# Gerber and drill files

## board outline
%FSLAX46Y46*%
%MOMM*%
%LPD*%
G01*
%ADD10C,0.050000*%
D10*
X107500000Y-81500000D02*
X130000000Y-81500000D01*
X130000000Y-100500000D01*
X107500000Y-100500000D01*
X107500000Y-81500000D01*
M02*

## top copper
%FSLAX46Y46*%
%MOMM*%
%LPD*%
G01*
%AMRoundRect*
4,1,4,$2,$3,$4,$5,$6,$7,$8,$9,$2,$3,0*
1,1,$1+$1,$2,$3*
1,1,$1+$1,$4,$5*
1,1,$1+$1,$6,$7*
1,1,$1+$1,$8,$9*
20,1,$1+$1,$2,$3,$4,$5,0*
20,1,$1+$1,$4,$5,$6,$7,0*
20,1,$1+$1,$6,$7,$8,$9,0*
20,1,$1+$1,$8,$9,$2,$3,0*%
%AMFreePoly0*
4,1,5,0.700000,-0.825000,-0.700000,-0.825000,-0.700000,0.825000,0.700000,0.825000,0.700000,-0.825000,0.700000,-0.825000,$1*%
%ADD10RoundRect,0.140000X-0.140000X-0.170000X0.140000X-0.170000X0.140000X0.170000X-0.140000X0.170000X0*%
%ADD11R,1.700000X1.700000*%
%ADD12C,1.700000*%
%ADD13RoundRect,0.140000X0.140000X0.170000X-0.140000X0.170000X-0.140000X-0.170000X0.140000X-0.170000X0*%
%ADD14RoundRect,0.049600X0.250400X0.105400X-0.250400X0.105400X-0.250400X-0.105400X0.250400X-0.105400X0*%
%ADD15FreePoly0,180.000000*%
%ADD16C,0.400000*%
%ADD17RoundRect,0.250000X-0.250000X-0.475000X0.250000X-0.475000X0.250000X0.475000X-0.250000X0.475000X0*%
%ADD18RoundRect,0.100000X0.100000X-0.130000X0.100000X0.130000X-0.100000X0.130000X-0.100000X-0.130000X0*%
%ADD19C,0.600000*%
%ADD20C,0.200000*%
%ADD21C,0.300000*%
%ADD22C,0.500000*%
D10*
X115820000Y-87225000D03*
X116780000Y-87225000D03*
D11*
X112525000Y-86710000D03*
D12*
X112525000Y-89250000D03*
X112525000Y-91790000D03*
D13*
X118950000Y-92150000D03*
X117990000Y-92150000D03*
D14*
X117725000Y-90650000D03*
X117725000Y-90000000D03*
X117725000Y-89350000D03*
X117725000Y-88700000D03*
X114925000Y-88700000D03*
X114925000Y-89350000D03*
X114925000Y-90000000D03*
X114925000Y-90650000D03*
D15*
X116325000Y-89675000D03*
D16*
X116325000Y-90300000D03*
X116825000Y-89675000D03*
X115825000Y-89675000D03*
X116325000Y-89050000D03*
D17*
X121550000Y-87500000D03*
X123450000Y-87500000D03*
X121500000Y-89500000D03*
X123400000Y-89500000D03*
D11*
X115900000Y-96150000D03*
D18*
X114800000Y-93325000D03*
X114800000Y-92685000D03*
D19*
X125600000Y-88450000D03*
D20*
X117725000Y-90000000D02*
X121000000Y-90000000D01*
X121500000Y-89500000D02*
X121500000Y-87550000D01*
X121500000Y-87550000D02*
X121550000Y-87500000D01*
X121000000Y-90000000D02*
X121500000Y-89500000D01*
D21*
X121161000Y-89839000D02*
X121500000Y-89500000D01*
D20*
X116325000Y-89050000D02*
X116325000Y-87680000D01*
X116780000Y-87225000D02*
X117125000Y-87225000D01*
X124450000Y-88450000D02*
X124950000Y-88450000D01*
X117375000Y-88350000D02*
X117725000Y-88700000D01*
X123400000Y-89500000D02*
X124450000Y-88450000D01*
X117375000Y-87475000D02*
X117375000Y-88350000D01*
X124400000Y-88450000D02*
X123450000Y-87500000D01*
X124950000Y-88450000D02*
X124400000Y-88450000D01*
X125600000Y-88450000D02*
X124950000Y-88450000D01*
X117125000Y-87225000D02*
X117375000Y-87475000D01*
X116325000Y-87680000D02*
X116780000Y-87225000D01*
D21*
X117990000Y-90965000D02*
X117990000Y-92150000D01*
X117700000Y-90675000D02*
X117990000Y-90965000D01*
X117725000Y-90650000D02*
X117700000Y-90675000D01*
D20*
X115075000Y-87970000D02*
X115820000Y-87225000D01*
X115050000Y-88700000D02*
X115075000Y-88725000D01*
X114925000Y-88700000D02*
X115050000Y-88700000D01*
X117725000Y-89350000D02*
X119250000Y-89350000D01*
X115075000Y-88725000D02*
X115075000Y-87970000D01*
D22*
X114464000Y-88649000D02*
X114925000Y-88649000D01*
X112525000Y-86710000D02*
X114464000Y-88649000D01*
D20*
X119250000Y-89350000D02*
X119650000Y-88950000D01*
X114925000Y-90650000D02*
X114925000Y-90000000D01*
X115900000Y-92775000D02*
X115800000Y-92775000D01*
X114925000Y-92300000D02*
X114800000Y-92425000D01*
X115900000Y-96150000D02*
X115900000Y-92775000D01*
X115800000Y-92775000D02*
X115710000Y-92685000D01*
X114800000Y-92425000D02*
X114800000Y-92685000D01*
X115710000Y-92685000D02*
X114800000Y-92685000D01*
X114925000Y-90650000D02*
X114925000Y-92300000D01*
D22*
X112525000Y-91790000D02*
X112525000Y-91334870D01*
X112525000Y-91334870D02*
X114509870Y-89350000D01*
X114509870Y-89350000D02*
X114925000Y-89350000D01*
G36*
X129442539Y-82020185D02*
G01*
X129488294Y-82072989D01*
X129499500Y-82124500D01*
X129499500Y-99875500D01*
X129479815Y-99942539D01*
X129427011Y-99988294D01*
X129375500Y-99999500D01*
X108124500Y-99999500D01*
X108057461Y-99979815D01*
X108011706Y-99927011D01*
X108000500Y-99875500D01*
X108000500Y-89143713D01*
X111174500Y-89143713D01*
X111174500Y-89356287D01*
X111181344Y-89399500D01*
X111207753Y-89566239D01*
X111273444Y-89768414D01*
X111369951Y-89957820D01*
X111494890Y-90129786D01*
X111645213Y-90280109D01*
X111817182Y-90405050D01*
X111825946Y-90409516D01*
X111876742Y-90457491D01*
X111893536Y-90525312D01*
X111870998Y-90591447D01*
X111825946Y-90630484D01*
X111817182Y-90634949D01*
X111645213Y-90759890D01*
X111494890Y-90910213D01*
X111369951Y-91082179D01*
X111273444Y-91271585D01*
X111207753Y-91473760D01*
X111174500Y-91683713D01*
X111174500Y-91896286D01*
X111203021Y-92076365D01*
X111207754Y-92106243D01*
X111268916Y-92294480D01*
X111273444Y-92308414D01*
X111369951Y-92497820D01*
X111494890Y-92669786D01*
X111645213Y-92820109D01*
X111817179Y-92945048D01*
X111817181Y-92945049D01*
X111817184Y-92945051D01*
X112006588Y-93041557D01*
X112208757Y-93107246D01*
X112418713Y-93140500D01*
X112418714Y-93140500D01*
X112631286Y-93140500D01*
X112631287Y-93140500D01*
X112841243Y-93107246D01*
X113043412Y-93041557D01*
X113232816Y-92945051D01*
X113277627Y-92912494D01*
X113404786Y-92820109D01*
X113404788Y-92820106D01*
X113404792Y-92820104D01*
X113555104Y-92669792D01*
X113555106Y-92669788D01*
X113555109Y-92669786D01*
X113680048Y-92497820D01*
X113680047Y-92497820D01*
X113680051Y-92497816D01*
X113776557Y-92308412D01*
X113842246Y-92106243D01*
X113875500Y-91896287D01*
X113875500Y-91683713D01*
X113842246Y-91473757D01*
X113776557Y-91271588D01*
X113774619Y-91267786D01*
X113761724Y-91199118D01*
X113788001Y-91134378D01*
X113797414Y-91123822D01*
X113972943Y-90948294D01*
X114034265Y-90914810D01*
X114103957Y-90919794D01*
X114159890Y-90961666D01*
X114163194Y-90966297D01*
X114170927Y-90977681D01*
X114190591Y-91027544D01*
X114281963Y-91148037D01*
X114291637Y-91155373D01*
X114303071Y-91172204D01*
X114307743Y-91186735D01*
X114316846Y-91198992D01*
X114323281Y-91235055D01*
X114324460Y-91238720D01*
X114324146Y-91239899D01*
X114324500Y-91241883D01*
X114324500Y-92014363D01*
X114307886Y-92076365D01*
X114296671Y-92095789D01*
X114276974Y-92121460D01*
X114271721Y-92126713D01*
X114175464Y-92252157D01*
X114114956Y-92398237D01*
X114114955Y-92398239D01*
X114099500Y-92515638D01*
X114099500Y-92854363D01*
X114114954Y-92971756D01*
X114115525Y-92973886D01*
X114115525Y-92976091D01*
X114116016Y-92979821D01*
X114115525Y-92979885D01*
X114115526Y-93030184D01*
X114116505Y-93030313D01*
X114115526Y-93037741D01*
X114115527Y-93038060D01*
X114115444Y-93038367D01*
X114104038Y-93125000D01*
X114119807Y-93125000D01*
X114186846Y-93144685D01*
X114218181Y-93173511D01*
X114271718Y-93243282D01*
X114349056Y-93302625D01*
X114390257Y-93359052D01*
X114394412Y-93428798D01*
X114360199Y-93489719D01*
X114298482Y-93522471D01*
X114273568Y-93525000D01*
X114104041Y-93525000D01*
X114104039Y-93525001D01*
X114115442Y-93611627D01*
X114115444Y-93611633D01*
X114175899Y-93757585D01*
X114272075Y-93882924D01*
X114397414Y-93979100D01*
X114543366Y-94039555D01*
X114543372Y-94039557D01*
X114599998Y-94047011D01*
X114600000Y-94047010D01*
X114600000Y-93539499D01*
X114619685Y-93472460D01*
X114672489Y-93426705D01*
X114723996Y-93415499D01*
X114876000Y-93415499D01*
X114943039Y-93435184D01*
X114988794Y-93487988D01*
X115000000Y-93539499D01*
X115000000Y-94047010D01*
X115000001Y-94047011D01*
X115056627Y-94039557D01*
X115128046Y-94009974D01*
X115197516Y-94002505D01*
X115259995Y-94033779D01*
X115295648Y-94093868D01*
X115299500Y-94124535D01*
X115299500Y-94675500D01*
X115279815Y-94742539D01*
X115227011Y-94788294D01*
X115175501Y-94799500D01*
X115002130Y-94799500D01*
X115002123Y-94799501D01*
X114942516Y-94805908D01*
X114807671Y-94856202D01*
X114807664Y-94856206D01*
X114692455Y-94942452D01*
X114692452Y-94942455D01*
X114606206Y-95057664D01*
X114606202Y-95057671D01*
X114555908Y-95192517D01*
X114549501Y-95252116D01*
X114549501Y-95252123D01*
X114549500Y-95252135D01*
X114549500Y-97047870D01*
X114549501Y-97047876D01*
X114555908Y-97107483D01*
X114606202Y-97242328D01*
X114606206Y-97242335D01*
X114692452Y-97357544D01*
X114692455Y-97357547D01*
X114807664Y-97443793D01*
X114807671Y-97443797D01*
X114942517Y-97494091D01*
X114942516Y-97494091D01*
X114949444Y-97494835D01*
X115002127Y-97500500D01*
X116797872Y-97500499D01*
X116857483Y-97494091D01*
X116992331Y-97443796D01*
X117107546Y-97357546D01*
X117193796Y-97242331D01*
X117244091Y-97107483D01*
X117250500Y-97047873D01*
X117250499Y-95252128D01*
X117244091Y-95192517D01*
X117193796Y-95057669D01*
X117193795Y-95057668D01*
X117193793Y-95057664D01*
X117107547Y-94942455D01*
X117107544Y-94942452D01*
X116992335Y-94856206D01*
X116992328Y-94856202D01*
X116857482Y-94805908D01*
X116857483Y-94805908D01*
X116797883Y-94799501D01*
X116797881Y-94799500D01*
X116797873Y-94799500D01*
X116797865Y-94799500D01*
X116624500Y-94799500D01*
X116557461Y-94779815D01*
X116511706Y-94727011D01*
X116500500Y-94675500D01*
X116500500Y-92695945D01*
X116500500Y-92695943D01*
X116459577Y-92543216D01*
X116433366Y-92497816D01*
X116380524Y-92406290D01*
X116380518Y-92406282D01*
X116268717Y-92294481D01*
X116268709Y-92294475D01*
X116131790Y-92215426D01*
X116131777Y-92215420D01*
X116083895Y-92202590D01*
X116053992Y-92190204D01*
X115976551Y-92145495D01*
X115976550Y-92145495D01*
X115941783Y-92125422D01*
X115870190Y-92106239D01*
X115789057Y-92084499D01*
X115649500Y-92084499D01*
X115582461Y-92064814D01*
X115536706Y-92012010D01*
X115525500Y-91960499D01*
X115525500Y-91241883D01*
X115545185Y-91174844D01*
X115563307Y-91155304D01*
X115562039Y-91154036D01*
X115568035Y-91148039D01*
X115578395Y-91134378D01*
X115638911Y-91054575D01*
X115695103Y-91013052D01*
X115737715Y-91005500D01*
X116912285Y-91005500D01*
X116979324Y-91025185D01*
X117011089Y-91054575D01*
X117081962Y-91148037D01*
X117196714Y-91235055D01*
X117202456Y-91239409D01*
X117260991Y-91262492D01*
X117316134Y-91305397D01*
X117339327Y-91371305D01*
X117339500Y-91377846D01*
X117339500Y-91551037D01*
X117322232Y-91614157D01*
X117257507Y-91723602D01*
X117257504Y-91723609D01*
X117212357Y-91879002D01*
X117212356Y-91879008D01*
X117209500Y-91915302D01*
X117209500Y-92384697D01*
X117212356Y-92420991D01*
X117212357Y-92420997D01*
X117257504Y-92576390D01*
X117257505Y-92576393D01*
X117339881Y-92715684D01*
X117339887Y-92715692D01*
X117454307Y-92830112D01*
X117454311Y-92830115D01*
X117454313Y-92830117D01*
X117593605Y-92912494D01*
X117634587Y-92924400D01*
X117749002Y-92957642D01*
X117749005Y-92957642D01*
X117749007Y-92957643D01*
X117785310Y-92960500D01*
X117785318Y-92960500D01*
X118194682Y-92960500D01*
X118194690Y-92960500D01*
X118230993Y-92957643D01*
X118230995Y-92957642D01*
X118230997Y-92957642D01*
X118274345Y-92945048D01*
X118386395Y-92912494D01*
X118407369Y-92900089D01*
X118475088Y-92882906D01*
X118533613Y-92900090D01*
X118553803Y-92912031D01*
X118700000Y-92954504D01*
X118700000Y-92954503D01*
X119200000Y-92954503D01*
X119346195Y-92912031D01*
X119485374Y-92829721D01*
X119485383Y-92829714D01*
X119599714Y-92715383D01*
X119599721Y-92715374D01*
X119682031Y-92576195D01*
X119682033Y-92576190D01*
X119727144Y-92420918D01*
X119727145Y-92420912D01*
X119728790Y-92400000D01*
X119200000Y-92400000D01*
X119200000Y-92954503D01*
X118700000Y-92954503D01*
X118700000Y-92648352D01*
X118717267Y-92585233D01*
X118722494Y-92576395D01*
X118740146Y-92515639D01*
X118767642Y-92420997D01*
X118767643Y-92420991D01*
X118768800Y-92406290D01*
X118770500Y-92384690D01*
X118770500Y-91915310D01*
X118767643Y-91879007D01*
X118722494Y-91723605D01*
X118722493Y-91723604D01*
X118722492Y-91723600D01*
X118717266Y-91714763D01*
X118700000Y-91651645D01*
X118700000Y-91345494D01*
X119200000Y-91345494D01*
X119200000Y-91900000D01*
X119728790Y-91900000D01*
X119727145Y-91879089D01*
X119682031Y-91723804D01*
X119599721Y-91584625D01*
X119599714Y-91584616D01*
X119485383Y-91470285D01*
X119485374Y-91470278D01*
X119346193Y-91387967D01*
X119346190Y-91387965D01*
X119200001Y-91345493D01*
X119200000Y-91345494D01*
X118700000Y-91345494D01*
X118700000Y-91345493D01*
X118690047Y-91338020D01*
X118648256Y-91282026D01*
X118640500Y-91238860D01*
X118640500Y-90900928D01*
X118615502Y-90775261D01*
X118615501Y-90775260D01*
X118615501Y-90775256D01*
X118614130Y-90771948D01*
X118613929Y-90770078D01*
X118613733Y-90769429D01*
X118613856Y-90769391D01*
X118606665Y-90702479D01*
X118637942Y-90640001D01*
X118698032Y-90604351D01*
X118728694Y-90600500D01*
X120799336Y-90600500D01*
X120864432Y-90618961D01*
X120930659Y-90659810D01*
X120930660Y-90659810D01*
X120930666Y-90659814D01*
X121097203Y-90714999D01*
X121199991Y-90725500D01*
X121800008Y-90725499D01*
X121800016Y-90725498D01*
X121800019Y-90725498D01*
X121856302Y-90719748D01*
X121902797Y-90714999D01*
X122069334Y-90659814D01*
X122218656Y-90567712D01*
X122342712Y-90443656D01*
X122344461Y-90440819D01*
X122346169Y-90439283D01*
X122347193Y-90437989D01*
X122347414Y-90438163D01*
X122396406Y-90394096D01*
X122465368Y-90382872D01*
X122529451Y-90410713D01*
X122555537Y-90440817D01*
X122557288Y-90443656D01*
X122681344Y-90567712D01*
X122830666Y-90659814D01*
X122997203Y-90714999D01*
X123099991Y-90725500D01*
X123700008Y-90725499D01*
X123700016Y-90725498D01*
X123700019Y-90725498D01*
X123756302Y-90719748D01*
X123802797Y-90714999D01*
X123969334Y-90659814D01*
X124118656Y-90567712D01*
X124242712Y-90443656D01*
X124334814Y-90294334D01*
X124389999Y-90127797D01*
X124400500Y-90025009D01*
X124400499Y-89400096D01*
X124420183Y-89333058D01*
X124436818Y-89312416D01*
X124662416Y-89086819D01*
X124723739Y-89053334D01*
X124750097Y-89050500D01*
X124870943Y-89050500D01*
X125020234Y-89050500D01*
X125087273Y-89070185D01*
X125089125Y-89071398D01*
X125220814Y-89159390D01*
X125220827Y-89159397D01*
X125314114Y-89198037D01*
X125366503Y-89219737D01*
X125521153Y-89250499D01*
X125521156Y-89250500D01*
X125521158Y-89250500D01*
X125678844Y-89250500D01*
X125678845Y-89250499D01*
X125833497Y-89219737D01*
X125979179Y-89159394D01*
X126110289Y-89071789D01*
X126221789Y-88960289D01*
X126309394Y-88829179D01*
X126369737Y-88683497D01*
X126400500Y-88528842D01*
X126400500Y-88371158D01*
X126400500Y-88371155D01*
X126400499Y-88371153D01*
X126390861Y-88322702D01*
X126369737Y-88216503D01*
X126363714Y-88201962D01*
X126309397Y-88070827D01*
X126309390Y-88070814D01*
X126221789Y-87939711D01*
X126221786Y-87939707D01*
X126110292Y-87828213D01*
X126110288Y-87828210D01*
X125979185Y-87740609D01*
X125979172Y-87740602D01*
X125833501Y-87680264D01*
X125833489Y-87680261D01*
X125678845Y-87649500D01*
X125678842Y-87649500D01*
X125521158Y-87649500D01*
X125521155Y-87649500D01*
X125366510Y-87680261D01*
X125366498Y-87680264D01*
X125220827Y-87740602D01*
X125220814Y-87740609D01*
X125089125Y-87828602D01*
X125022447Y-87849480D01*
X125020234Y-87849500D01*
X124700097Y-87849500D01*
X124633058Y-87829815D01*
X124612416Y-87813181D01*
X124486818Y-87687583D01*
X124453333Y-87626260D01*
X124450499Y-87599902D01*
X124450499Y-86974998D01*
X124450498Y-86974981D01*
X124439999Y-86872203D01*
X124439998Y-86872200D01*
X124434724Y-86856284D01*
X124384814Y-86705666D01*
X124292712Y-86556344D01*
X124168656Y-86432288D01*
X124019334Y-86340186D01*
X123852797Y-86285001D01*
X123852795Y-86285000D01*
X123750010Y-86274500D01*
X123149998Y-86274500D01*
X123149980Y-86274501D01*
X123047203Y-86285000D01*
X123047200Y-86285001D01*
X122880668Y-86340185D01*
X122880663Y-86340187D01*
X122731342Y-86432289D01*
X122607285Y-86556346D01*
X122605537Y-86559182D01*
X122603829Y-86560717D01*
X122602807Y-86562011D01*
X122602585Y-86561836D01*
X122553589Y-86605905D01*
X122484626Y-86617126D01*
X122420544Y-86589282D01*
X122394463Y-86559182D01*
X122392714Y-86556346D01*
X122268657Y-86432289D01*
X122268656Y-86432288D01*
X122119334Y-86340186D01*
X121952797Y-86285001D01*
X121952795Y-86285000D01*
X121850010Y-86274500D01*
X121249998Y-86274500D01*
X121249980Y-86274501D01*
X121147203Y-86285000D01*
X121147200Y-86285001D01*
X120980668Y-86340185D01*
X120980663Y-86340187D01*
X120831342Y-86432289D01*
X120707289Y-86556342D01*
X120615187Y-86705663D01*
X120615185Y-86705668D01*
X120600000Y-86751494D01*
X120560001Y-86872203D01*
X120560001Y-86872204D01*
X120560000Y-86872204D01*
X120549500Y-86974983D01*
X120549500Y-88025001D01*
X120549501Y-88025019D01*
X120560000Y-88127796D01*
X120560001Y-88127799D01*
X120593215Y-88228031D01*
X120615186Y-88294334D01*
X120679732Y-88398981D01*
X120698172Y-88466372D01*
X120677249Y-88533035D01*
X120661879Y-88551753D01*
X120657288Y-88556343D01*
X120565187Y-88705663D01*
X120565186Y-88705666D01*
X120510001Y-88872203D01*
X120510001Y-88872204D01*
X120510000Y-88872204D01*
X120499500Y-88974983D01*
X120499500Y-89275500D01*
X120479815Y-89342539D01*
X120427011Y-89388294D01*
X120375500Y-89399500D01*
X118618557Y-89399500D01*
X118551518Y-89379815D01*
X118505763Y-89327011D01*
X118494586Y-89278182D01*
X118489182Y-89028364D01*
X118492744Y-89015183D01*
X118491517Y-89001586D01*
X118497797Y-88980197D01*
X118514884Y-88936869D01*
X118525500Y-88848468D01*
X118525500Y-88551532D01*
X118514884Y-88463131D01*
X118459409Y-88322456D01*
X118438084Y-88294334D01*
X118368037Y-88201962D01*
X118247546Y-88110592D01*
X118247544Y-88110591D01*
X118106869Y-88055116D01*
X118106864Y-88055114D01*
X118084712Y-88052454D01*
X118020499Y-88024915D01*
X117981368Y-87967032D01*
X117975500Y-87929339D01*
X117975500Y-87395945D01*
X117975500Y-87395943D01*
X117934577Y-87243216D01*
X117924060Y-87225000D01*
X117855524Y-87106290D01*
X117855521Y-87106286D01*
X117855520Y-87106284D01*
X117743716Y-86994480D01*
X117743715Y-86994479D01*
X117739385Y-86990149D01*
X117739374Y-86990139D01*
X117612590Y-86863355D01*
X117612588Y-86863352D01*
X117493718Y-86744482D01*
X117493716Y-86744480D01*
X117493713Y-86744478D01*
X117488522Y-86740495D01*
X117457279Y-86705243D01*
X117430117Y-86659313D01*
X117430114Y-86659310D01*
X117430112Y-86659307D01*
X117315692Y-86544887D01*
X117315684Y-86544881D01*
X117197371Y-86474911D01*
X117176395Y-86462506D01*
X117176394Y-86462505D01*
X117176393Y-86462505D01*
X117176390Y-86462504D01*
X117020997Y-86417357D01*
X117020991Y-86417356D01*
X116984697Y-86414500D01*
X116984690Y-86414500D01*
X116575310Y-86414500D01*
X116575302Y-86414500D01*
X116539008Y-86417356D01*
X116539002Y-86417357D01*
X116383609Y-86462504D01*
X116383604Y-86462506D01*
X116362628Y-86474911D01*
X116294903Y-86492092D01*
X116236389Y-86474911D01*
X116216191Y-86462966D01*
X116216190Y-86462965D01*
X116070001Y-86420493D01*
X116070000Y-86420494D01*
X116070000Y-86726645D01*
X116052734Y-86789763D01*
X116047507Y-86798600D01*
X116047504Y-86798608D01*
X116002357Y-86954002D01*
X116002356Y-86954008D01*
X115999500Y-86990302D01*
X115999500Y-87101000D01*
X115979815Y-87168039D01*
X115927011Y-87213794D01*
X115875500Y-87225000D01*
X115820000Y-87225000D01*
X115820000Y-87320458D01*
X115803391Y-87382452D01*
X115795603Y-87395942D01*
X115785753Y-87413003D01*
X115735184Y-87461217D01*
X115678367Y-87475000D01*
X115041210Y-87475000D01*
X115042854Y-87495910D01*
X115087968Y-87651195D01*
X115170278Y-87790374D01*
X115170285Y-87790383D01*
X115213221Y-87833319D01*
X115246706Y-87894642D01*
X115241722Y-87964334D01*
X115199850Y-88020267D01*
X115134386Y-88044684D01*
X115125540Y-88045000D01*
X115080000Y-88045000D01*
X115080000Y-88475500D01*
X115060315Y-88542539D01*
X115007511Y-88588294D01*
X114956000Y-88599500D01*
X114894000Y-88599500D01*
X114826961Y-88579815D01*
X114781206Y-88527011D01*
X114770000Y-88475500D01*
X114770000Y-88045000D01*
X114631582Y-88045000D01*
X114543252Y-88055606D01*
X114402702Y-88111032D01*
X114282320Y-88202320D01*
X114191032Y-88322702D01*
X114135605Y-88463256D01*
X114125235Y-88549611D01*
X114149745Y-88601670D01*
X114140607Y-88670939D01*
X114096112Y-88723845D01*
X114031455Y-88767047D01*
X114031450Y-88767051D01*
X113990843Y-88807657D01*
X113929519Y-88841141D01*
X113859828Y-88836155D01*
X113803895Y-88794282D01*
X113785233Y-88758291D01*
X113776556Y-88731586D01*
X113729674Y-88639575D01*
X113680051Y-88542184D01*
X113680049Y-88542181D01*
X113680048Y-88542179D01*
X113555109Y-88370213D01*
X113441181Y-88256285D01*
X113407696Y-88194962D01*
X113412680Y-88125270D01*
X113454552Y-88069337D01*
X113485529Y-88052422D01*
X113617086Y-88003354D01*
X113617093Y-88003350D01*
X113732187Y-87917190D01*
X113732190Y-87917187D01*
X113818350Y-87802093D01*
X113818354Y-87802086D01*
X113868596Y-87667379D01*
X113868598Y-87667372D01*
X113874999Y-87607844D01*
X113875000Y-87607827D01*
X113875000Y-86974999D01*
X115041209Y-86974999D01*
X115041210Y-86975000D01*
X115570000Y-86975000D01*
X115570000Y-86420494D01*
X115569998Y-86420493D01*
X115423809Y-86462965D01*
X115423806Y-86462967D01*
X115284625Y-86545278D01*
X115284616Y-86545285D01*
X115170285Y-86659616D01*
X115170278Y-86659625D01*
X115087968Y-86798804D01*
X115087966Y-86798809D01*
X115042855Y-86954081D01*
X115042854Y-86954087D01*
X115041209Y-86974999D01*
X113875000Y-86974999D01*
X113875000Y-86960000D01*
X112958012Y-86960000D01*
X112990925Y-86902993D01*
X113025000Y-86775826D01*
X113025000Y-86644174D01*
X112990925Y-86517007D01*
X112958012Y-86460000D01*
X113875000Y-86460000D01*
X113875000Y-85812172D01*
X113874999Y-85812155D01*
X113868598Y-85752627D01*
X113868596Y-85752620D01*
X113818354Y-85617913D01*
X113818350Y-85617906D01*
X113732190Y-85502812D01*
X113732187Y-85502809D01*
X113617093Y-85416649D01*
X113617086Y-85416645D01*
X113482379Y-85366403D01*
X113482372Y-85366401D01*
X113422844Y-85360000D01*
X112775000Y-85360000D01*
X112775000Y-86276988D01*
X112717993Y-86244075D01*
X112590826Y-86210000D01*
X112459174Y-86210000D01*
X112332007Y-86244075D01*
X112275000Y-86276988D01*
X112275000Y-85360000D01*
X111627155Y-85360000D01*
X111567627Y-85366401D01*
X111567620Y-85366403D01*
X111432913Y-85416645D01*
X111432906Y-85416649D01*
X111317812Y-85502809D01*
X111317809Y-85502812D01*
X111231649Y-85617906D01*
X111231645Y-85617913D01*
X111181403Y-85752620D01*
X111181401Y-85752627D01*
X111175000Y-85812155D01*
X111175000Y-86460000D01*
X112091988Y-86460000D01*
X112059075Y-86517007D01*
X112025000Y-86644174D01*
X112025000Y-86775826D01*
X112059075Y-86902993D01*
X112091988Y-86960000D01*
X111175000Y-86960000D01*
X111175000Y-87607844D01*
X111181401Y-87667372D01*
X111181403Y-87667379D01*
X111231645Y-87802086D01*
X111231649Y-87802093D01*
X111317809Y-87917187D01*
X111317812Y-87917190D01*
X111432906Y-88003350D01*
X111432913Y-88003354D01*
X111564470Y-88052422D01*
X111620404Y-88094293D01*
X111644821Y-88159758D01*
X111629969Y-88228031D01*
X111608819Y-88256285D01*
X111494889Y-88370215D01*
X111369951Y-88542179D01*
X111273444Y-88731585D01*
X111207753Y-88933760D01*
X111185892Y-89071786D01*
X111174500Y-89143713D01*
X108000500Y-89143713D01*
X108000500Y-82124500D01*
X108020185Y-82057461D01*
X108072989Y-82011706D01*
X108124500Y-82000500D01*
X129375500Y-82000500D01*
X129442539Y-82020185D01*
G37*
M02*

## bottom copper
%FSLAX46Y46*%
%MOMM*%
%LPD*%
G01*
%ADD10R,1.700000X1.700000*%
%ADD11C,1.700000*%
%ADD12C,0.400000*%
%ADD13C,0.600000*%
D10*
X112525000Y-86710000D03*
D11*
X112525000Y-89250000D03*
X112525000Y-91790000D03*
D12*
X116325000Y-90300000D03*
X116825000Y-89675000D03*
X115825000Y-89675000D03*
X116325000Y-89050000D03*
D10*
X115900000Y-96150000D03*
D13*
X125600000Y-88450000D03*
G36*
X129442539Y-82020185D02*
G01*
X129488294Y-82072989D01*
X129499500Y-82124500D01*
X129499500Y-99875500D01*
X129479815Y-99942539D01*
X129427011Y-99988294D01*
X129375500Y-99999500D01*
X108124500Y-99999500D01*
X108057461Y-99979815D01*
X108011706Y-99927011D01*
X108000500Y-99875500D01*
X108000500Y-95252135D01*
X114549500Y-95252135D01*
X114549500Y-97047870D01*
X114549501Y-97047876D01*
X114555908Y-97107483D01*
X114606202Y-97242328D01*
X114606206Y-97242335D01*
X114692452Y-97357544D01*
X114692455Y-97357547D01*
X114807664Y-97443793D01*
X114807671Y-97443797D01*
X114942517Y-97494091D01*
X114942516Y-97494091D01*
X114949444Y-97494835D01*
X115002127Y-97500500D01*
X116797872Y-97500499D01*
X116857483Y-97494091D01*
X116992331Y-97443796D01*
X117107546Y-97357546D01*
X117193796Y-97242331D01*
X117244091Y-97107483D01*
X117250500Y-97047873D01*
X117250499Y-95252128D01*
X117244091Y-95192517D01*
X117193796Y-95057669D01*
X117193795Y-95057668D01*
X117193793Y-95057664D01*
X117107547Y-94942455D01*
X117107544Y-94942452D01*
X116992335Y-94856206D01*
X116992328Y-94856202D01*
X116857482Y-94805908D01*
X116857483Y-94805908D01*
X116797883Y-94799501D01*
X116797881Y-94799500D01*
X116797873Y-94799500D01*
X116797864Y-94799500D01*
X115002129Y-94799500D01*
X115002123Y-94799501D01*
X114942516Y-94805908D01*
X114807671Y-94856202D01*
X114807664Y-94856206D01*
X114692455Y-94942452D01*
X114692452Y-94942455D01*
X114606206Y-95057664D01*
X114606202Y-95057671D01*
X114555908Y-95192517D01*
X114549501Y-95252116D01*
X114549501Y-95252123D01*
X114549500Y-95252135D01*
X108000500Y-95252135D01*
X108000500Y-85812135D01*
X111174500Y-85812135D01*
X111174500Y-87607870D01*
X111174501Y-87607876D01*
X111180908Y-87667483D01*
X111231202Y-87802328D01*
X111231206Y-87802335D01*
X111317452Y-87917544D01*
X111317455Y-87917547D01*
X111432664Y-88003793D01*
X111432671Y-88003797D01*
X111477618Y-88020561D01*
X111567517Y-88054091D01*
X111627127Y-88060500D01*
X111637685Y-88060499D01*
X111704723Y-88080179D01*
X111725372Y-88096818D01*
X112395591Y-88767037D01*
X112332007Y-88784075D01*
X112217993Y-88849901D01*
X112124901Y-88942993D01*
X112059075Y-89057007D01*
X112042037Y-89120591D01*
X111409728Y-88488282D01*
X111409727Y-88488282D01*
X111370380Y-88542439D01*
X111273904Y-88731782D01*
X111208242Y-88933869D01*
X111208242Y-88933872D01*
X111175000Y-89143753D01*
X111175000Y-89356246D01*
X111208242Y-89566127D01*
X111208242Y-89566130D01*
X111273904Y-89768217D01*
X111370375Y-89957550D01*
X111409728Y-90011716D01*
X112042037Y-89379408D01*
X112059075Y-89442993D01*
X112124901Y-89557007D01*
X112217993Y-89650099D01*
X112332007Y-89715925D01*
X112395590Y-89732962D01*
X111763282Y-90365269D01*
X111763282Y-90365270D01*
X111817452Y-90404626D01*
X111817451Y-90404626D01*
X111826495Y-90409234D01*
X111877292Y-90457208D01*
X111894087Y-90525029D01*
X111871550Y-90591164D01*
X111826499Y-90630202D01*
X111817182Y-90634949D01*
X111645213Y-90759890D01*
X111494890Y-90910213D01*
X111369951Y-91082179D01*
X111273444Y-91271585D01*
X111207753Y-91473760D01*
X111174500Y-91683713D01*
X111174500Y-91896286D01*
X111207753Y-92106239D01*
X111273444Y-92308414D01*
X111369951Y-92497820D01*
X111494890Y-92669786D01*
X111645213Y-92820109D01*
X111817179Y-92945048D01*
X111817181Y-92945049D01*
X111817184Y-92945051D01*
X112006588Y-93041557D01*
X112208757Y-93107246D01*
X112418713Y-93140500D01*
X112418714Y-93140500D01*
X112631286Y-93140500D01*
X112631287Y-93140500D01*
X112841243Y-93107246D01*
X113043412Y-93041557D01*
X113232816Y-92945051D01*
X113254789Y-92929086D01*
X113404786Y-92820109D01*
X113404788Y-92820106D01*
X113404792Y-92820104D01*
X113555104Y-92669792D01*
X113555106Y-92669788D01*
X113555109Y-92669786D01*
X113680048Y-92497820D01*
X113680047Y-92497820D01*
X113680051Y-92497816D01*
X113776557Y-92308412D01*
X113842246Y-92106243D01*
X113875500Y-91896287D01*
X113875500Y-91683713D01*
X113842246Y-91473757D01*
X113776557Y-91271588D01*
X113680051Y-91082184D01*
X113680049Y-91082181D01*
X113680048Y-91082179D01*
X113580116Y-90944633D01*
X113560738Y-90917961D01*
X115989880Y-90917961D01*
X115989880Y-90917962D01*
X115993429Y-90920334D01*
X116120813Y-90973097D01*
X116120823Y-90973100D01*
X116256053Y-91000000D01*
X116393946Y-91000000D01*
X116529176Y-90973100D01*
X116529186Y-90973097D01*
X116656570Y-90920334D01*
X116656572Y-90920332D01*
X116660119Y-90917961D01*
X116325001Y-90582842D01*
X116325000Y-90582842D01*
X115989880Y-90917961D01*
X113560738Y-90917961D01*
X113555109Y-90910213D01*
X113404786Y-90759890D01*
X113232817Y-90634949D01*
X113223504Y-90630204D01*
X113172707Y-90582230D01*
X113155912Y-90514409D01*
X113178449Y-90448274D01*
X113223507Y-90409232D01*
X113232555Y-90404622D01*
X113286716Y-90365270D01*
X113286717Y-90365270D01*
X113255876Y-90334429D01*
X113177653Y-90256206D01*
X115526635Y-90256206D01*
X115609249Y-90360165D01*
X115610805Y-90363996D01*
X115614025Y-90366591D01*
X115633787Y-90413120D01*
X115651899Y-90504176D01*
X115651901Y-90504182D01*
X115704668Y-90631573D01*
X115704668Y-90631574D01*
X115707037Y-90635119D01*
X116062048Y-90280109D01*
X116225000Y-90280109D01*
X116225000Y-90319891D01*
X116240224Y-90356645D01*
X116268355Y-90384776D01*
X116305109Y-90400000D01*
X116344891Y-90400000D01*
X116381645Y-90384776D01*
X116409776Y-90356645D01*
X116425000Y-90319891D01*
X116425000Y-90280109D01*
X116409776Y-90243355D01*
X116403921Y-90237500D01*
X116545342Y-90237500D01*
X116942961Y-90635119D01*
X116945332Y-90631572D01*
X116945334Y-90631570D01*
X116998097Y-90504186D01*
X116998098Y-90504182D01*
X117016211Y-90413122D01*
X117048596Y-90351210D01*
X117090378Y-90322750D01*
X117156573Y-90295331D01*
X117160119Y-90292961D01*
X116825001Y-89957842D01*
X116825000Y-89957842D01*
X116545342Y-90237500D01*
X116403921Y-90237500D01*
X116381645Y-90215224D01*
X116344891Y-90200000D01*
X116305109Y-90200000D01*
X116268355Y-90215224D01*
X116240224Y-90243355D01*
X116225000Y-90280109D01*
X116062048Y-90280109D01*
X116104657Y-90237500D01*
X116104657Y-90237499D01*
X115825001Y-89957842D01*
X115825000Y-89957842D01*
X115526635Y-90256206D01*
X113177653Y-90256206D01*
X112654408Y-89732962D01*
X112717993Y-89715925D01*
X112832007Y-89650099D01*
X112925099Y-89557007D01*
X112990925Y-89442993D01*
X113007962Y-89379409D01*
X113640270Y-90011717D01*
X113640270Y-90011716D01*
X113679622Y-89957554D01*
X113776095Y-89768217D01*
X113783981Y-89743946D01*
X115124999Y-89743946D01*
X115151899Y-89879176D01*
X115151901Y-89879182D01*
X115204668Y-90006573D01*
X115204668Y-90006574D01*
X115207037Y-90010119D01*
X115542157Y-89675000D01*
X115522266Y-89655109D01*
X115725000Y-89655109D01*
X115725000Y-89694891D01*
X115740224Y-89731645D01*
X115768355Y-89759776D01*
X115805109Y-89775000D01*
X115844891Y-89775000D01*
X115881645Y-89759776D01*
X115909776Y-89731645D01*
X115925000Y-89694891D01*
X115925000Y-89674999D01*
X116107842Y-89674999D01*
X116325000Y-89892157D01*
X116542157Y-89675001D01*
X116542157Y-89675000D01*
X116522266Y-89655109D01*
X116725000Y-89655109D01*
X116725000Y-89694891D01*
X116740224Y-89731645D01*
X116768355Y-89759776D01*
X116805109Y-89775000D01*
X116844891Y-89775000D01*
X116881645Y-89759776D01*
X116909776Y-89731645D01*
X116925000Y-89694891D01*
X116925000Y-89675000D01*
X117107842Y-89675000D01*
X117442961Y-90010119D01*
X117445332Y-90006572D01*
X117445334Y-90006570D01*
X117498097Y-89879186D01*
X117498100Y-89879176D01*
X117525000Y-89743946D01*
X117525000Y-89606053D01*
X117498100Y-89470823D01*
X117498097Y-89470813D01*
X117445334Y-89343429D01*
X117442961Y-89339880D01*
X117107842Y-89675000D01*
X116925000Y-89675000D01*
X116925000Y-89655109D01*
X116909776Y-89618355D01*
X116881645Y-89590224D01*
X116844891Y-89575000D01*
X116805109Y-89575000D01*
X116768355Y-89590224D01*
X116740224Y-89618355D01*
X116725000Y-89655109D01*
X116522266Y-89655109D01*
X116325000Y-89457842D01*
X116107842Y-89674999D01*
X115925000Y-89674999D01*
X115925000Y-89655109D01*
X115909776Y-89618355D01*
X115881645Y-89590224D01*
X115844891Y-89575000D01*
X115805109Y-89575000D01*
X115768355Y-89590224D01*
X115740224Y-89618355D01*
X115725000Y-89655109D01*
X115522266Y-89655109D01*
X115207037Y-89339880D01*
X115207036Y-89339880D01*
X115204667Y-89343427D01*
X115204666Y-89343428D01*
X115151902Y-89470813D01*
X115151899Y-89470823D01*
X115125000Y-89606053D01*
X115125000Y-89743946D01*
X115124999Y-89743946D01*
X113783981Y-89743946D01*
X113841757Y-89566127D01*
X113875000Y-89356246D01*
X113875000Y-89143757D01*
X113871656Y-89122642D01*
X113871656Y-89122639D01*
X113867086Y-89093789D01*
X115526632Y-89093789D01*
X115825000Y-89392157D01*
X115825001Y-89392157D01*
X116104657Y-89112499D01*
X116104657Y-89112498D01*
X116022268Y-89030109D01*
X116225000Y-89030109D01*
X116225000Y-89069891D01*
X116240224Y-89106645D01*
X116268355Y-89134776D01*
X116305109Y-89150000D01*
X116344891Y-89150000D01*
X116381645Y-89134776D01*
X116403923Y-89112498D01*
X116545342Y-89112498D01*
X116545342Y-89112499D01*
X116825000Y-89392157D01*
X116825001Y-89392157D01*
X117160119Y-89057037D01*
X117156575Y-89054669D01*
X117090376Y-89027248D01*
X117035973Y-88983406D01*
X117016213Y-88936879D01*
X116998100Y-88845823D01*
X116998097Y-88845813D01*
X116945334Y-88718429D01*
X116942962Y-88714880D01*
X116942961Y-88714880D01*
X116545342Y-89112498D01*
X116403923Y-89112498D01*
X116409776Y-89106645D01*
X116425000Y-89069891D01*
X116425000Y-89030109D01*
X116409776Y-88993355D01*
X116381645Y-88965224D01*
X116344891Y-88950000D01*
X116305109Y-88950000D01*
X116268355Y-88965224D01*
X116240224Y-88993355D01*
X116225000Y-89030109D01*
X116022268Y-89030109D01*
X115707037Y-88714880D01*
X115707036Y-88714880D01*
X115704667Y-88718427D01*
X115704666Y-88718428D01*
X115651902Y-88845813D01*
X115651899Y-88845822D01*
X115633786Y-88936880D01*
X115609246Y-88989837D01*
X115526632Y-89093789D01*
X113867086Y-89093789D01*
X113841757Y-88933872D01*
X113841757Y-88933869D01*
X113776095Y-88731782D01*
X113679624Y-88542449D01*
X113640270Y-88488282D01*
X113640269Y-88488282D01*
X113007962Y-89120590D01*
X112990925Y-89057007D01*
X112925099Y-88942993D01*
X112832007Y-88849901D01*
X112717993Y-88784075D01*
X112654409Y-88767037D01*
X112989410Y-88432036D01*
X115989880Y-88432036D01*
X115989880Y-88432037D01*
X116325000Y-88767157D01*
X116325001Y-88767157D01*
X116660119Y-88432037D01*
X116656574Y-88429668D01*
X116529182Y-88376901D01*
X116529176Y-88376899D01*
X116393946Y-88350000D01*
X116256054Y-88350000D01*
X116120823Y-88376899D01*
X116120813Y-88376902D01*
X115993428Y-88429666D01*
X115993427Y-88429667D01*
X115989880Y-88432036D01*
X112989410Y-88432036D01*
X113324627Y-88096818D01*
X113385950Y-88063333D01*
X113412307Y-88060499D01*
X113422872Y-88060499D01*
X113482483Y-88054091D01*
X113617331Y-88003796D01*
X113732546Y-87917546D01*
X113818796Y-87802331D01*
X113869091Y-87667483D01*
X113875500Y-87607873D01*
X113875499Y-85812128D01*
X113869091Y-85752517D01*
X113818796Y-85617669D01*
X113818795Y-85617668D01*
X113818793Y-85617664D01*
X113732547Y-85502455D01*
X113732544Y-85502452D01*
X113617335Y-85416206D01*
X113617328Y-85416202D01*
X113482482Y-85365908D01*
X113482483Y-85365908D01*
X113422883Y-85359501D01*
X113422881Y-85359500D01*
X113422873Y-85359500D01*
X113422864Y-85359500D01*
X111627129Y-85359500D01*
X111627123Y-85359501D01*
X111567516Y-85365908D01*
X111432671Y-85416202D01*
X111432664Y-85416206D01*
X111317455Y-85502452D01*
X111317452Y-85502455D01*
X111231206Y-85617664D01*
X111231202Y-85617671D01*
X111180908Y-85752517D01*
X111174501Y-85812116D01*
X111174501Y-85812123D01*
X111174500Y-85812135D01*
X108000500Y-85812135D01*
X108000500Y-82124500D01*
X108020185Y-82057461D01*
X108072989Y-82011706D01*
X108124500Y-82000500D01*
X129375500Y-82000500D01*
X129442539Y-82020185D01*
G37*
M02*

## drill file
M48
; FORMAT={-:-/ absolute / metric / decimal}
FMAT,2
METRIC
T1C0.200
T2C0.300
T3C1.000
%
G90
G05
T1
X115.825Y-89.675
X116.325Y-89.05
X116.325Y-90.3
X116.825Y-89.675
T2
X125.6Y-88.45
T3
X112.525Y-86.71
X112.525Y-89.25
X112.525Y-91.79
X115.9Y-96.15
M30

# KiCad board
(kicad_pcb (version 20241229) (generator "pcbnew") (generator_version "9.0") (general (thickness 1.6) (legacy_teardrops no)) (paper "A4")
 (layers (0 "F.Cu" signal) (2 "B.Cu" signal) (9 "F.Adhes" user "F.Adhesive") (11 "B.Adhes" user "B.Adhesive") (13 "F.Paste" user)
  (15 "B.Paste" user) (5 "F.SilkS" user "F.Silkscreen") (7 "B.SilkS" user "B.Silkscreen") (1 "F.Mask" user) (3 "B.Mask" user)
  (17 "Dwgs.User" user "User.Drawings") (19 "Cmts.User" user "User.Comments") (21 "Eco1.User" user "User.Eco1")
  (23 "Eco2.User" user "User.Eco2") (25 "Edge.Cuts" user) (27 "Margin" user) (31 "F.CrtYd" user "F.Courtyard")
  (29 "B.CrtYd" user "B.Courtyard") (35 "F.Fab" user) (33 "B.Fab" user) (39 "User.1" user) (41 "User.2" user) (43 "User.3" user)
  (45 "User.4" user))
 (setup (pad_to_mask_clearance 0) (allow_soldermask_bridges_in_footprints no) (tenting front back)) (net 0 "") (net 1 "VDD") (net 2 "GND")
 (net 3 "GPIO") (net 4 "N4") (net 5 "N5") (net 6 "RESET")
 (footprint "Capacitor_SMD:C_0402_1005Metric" (layer "F.Cu") (at 116.3 87.225)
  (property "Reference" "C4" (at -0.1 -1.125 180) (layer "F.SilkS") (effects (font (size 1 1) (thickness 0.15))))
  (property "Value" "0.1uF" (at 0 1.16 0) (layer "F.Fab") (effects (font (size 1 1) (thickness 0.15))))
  (pad "1" smd roundrect (at -0.48 0) (size 0.56 0.62) (layers "F.Cu" "F.Mask" "F.Paste") (roundrect_rratio 0.25) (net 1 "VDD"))
  (pad "2" smd roundrect (at 0.48 0) (size 0.56 0.62) (layers "F.Cu" "F.Mask" "F.Paste") (roundrect_rratio 0.25) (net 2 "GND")))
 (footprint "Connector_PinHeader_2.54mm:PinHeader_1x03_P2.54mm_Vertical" (layer "F.Cu") (at 112.525 86.71)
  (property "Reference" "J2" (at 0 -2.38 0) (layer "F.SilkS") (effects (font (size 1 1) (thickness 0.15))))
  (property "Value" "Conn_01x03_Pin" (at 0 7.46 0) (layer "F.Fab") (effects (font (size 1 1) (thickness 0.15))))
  (pad "1" thru_hole rect (at 0 0) (size 1.7 1.7) (drill 1) (layers "*.Cu" "*.Mask") (remove_unused_layers no) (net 1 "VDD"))
  (pad "2" thru_hole circle (at 0 2.54) (size 1.7 1.7) (drill 1) (layers "*.Cu" "*.Mask") (remove_unused_layers no) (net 2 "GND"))
  (pad "3" thru_hole circle (at 0 5.08) (size 1.7 1.7) (drill 1) (layers "*.Cu" "*.Mask") (remove_unused_layers no) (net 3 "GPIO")))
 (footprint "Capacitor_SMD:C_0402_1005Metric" (layer "F.Cu") (at 118.47 92.15 180)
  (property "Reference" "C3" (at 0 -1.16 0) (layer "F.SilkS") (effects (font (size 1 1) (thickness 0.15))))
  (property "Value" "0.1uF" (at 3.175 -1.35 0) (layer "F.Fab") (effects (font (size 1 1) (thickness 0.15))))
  (pad "1" smd roundrect (at -0.48 0 180) (size 0.56 0.62) (layers "F.Cu" "F.Mask" "F.Paste") (roundrect_rratio 0.25) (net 1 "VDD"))
  (pad "2" smd roundrect (at 0.48 0 180) (size 0.56 0.62) (layers "F.Cu" "F.Mask" "F.Paste") (roundrect_rratio 0.25) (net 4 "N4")))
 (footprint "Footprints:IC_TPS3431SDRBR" (layer "F.Cu") (at 116.325 89.675 180)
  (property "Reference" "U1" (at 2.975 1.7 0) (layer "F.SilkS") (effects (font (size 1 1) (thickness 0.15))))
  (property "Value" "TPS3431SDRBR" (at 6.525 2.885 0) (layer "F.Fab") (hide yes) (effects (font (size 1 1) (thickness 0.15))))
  (pad "1" smd roundrect (at -1.4 -0.975 180) (size 0.6 0.31) (layers "F.Cu" "F.Paste") (roundrect_rratio 0.16) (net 4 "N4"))
  (pad "2" smd roundrect (at -1.4 -0.325 180) (size 0.6 0.31) (layers "F.Cu" "F.Paste") (roundrect_rratio 0.16) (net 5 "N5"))
  (pad "3" smd roundrect (at -1.4 0.325 180) (size 0.6 0.31) (layers "F.Cu" "F.Paste") (roundrect_rratio 0.16) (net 1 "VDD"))
  (pad "4" smd roundrect (at -1.4 0.975 180) (size 0.6 0.31) (layers "F.Cu" "F.Paste") (roundrect_rratio 0.16) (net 2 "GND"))
  (pad "5" smd roundrect (at 1.4 0.975 180) (size 0.6 0.31) (layers "F.Cu" "F.Paste") (roundrect_rratio 0.16) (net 1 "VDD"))
  (pad "6" smd roundrect (at 1.4 0.325 180) (size 0.6 0.31) (layers "F.Cu" "F.Paste") (roundrect_rratio 0.16) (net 3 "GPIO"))
  (pad "7" smd roundrect (at 1.4 -0.325 180) (size 0.6 0.31) (layers "F.Cu" "F.Paste") (roundrect_rratio 0.16) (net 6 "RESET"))
  (pad "8" smd roundrect (at 1.4 -0.975 180) (size 0.6 0.31) (layers "F.Cu" "F.Paste") (roundrect_rratio 0.16) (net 6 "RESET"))
  (pad "9" smd custom (at 0 0 180) (size 1.4 1.65) (layers "F.Cu") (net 2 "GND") (options (clearance outline) (anchor rect)) (primitives))
  (pad "10" thru_hole circle (at 0 -0.625 180) (size 0.4 0.4) (drill 0.2) (layers "*.Cu") (remove_unused_layers no) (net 2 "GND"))
  (pad "11" thru_hole circle (at -0.5 0 180) (size 0.4 0.4) (drill 0.2) (layers "*.Cu") (remove_unused_layers no) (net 2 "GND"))
  (pad "12" thru_hole circle (at 0.5 0 180) (size 0.4 0.4) (drill 0.2) (layers "*.Cu") (remove_unused_layers no) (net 2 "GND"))
  (pad "13" thru_hole circle (at 0 0.625 180) (size 0.4 0.4) (drill 0.2) (layers "*.Cu") (remove_unused_layers no) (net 2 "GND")))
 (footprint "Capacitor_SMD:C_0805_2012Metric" (layer "F.Cu") (at 122.5 87.5)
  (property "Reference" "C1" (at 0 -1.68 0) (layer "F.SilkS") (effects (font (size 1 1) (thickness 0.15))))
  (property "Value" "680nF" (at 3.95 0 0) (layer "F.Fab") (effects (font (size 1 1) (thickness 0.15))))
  (pad "1" smd roundrect (at -0.95 0) (size 1 1.45) (layers "F.Cu" "F.Mask" "F.Paste") (roundrect_rratio 0.25) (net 5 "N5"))
  (pad "2" smd roundrect (at 0.95 0) (size 1 1.45) (layers "F.Cu" "F.Mask" "F.Paste") (roundrect_rratio 0.25) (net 2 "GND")))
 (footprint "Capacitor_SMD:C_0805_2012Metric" (layer "F.Cu") (at 122.45 89.5)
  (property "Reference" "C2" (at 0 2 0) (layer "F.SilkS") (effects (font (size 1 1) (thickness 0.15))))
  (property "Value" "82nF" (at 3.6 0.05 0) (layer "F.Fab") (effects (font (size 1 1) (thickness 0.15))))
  (pad "1" smd roundrect (at -0.95 0) (size 1 1.45) (layers "F.Cu" "F.Mask" "F.Paste") (roundrect_rratio 0.25) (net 5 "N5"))
  (pad "2" smd roundrect (at 0.95 0) (size 1 1.45) (layers "F.Cu" "F.Mask" "F.Paste") (roundrect_rratio 0.25) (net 2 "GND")))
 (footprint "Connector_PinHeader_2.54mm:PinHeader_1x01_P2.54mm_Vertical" (layer "F.Cu") (at 115.9 96.15)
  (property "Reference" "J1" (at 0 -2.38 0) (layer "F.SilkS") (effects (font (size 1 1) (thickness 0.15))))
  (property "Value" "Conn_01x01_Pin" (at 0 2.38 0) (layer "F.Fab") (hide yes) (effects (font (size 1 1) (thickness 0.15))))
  (pad "1" thru_hole rect (at 0 0) (size 1.7 1.7) (drill 1) (layers "*.Cu" "*.Mask") (remove_unused_layers no) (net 6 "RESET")))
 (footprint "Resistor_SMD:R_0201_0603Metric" (layer "F.Cu") (at 114.8 93.005 90)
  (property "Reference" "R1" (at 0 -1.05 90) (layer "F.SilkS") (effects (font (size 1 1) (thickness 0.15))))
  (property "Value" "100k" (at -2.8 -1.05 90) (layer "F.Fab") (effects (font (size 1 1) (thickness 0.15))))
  (pad "" smd roundrect (at -0.345 0 90) (size 0.318 0.36) (layers "F.Paste") (roundrect_rratio 0.25))
  (pad "" smd roundrect (at 0.345 0 90) (size 0.318 0.36) (layers "F.Paste") (roundrect_rratio 0.25))
  (pad "1" smd roundrect (at -0.32 0 90) (size 0.46 0.4) (layers "F.Cu" "F.Mask") (roundrect_rratio 0.25) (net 1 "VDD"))
  (pad "2" smd roundrect (at 0.32 0 90) (size 0.46 0.4) (layers "F.Cu" "F.Mask") (roundrect_rratio 0.25) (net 6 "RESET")))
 (gr_rect (start 107.5 81.5) (end 130 100.5) (stroke (width 0.05) (type default)) (fill no) (layer "Edge.Cuts"))
 (segment (start 117.725 90) (end 121 90) (width 0.2) (layer "F.Cu") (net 5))
 (segment (start 121.5 89.5) (end 121.5 87.55) (width 0.2) (layer "F.Cu") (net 5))
 (segment (start 121.5 87.55) (end 121.55 87.5) (width 0.2) (layer "F.Cu") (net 5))
 (segment (start 121 90) (end 121.5 89.5) (width 0.2) (layer "F.Cu") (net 5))
 (segment (start 121.161 89.839) (end 121.5 89.5) (width 0.3) (layer "F.Cu") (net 5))
 (segment (start 116.325 89.05) (end 116.325 87.68) (width 0.2) (layer "F.Cu") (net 2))
 (segment (start 116.78 87.225) (end 117.125 87.225) (width 0.2) (layer "F.Cu") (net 2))
 (segment (start 124.45 88.45) (end 124.95 88.45) (width 0.2) (layer "F.Cu") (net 2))
 (segment (start 117.375 88.35) (end 117.725 88.7) (width 0.2) (layer "F.Cu") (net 2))
 (segment (start 123.4 89.5) (end 124.45 88.45) (width 0.2) (layer "F.Cu") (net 2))
 (segment (start 117.375 87.475) (end 117.375 88.35) (width 0.2) (layer "F.Cu") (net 2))
 (segment (start 124.4 88.45) (end 123.45 87.5) (width 0.2) (layer "F.Cu") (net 2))
 (segment (start 124.95 88.45) (end 124.4 88.45) (width 0.2) (layer "F.Cu") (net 2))
 (segment (start 125.6 88.45) (end 124.95 88.45) (width 0.2) (layer "F.Cu") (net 2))
 (segment (start 117.125 87.225) (end 117.375 87.475) (width 0.2) (layer "F.Cu") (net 2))
 (segment (start 116.325 87.68) (end 116.78 87.225) (width 0.2) (layer "F.Cu") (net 2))
 (via (at 125.6 88.45) (size 0.6) (drill 0.3) (layers "F.Cu" "B.Cu") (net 2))
 (segment (start 117.99 90.965) (end 117.99 92.15) (width 0.3) (layer "F.Cu") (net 4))
 (segment (start 117.7 90.675) (end 117.99 90.965) (width 0.3) (layer "F.Cu") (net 4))
 (segment (start 117.725 90.65) (end 117.7 90.675) (width 0.3) (layer "F.Cu") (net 4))
 (segment (start 115.075 87.97) (end 115.82 87.225) (width 0.2) (layer "F.Cu") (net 1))
 (segment (start 115.05 88.7) (end 115.075 88.725) (width 0.2) (layer "F.Cu") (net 1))
 (segment (start 114.925 88.7) (end 115.05 88.7) (width 0.2) (layer "F.Cu") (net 1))
 (segment (start 117.725 89.35) (end 119.25 89.35) (width 0.2) (layer "F.Cu") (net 1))
 (segment (start 115.075 88.725) (end 115.075 87.97) (width 0.2) (layer "F.Cu") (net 1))
 (segment (start 114.464 88.649) (end 114.925 88.649) (width 0.5) (layer "F.Cu") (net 1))
 (segment (start 112.525 86.71) (end 114.464 88.649) (width 0.5) (layer "F.Cu") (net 1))
 (segment (start 119.25 89.35) (end 119.65 88.95) (width 0.2) (layer "F.Cu") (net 1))
 (segment (start 114.925 90.65) (end 114.925 90) (width 0.2) (layer "F.Cu") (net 6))
 (segment (start 115.9 92.775) (end 115.8 92.775) (width 0.2) (layer "F.Cu") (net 6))
 (segment (start 114.925 92.3) (end 114.8 92.425) (width 0.2) (layer "F.Cu") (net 6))
 (segment (start 115.9 96.15) (end 115.9 92.775) (width 0.2) (layer "F.Cu") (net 6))
 (segment (start 115.8 92.775) (end 115.71 92.685) (width 0.2) (layer "F.Cu") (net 6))
 (segment (start 114.8 92.425) (end 114.8 92.685) (width 0.2) (layer "F.Cu") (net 6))
 (segment (start 115.71 92.685) (end 114.8 92.685) (width 0.2) (layer "F.Cu") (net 6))
 (segment (start 114.925 90.65) (end 114.925 92.3) (width 0.2) (layer "F.Cu") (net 6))
 (segment (start 112.525 91.79) (end 112.525 91.33487) (width 0.5) (layer "F.Cu") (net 3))
 (segment (start 112.525 91.33487) (end 114.50987 89.35) (width 0.5) (layer "F.Cu") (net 3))
 (segment (start 114.50987 89.35) (end 114.925 89.35) (width 0.5) (layer "F.Cu") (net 3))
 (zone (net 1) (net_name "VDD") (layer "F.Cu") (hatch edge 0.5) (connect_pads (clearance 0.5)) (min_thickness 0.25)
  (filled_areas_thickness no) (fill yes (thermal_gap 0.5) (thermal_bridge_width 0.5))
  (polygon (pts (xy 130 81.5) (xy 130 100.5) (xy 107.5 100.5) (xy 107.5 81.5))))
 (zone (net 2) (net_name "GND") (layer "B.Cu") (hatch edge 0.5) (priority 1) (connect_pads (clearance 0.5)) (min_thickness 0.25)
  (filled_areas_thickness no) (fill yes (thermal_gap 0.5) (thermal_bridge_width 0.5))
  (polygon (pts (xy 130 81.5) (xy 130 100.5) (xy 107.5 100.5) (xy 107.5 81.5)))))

